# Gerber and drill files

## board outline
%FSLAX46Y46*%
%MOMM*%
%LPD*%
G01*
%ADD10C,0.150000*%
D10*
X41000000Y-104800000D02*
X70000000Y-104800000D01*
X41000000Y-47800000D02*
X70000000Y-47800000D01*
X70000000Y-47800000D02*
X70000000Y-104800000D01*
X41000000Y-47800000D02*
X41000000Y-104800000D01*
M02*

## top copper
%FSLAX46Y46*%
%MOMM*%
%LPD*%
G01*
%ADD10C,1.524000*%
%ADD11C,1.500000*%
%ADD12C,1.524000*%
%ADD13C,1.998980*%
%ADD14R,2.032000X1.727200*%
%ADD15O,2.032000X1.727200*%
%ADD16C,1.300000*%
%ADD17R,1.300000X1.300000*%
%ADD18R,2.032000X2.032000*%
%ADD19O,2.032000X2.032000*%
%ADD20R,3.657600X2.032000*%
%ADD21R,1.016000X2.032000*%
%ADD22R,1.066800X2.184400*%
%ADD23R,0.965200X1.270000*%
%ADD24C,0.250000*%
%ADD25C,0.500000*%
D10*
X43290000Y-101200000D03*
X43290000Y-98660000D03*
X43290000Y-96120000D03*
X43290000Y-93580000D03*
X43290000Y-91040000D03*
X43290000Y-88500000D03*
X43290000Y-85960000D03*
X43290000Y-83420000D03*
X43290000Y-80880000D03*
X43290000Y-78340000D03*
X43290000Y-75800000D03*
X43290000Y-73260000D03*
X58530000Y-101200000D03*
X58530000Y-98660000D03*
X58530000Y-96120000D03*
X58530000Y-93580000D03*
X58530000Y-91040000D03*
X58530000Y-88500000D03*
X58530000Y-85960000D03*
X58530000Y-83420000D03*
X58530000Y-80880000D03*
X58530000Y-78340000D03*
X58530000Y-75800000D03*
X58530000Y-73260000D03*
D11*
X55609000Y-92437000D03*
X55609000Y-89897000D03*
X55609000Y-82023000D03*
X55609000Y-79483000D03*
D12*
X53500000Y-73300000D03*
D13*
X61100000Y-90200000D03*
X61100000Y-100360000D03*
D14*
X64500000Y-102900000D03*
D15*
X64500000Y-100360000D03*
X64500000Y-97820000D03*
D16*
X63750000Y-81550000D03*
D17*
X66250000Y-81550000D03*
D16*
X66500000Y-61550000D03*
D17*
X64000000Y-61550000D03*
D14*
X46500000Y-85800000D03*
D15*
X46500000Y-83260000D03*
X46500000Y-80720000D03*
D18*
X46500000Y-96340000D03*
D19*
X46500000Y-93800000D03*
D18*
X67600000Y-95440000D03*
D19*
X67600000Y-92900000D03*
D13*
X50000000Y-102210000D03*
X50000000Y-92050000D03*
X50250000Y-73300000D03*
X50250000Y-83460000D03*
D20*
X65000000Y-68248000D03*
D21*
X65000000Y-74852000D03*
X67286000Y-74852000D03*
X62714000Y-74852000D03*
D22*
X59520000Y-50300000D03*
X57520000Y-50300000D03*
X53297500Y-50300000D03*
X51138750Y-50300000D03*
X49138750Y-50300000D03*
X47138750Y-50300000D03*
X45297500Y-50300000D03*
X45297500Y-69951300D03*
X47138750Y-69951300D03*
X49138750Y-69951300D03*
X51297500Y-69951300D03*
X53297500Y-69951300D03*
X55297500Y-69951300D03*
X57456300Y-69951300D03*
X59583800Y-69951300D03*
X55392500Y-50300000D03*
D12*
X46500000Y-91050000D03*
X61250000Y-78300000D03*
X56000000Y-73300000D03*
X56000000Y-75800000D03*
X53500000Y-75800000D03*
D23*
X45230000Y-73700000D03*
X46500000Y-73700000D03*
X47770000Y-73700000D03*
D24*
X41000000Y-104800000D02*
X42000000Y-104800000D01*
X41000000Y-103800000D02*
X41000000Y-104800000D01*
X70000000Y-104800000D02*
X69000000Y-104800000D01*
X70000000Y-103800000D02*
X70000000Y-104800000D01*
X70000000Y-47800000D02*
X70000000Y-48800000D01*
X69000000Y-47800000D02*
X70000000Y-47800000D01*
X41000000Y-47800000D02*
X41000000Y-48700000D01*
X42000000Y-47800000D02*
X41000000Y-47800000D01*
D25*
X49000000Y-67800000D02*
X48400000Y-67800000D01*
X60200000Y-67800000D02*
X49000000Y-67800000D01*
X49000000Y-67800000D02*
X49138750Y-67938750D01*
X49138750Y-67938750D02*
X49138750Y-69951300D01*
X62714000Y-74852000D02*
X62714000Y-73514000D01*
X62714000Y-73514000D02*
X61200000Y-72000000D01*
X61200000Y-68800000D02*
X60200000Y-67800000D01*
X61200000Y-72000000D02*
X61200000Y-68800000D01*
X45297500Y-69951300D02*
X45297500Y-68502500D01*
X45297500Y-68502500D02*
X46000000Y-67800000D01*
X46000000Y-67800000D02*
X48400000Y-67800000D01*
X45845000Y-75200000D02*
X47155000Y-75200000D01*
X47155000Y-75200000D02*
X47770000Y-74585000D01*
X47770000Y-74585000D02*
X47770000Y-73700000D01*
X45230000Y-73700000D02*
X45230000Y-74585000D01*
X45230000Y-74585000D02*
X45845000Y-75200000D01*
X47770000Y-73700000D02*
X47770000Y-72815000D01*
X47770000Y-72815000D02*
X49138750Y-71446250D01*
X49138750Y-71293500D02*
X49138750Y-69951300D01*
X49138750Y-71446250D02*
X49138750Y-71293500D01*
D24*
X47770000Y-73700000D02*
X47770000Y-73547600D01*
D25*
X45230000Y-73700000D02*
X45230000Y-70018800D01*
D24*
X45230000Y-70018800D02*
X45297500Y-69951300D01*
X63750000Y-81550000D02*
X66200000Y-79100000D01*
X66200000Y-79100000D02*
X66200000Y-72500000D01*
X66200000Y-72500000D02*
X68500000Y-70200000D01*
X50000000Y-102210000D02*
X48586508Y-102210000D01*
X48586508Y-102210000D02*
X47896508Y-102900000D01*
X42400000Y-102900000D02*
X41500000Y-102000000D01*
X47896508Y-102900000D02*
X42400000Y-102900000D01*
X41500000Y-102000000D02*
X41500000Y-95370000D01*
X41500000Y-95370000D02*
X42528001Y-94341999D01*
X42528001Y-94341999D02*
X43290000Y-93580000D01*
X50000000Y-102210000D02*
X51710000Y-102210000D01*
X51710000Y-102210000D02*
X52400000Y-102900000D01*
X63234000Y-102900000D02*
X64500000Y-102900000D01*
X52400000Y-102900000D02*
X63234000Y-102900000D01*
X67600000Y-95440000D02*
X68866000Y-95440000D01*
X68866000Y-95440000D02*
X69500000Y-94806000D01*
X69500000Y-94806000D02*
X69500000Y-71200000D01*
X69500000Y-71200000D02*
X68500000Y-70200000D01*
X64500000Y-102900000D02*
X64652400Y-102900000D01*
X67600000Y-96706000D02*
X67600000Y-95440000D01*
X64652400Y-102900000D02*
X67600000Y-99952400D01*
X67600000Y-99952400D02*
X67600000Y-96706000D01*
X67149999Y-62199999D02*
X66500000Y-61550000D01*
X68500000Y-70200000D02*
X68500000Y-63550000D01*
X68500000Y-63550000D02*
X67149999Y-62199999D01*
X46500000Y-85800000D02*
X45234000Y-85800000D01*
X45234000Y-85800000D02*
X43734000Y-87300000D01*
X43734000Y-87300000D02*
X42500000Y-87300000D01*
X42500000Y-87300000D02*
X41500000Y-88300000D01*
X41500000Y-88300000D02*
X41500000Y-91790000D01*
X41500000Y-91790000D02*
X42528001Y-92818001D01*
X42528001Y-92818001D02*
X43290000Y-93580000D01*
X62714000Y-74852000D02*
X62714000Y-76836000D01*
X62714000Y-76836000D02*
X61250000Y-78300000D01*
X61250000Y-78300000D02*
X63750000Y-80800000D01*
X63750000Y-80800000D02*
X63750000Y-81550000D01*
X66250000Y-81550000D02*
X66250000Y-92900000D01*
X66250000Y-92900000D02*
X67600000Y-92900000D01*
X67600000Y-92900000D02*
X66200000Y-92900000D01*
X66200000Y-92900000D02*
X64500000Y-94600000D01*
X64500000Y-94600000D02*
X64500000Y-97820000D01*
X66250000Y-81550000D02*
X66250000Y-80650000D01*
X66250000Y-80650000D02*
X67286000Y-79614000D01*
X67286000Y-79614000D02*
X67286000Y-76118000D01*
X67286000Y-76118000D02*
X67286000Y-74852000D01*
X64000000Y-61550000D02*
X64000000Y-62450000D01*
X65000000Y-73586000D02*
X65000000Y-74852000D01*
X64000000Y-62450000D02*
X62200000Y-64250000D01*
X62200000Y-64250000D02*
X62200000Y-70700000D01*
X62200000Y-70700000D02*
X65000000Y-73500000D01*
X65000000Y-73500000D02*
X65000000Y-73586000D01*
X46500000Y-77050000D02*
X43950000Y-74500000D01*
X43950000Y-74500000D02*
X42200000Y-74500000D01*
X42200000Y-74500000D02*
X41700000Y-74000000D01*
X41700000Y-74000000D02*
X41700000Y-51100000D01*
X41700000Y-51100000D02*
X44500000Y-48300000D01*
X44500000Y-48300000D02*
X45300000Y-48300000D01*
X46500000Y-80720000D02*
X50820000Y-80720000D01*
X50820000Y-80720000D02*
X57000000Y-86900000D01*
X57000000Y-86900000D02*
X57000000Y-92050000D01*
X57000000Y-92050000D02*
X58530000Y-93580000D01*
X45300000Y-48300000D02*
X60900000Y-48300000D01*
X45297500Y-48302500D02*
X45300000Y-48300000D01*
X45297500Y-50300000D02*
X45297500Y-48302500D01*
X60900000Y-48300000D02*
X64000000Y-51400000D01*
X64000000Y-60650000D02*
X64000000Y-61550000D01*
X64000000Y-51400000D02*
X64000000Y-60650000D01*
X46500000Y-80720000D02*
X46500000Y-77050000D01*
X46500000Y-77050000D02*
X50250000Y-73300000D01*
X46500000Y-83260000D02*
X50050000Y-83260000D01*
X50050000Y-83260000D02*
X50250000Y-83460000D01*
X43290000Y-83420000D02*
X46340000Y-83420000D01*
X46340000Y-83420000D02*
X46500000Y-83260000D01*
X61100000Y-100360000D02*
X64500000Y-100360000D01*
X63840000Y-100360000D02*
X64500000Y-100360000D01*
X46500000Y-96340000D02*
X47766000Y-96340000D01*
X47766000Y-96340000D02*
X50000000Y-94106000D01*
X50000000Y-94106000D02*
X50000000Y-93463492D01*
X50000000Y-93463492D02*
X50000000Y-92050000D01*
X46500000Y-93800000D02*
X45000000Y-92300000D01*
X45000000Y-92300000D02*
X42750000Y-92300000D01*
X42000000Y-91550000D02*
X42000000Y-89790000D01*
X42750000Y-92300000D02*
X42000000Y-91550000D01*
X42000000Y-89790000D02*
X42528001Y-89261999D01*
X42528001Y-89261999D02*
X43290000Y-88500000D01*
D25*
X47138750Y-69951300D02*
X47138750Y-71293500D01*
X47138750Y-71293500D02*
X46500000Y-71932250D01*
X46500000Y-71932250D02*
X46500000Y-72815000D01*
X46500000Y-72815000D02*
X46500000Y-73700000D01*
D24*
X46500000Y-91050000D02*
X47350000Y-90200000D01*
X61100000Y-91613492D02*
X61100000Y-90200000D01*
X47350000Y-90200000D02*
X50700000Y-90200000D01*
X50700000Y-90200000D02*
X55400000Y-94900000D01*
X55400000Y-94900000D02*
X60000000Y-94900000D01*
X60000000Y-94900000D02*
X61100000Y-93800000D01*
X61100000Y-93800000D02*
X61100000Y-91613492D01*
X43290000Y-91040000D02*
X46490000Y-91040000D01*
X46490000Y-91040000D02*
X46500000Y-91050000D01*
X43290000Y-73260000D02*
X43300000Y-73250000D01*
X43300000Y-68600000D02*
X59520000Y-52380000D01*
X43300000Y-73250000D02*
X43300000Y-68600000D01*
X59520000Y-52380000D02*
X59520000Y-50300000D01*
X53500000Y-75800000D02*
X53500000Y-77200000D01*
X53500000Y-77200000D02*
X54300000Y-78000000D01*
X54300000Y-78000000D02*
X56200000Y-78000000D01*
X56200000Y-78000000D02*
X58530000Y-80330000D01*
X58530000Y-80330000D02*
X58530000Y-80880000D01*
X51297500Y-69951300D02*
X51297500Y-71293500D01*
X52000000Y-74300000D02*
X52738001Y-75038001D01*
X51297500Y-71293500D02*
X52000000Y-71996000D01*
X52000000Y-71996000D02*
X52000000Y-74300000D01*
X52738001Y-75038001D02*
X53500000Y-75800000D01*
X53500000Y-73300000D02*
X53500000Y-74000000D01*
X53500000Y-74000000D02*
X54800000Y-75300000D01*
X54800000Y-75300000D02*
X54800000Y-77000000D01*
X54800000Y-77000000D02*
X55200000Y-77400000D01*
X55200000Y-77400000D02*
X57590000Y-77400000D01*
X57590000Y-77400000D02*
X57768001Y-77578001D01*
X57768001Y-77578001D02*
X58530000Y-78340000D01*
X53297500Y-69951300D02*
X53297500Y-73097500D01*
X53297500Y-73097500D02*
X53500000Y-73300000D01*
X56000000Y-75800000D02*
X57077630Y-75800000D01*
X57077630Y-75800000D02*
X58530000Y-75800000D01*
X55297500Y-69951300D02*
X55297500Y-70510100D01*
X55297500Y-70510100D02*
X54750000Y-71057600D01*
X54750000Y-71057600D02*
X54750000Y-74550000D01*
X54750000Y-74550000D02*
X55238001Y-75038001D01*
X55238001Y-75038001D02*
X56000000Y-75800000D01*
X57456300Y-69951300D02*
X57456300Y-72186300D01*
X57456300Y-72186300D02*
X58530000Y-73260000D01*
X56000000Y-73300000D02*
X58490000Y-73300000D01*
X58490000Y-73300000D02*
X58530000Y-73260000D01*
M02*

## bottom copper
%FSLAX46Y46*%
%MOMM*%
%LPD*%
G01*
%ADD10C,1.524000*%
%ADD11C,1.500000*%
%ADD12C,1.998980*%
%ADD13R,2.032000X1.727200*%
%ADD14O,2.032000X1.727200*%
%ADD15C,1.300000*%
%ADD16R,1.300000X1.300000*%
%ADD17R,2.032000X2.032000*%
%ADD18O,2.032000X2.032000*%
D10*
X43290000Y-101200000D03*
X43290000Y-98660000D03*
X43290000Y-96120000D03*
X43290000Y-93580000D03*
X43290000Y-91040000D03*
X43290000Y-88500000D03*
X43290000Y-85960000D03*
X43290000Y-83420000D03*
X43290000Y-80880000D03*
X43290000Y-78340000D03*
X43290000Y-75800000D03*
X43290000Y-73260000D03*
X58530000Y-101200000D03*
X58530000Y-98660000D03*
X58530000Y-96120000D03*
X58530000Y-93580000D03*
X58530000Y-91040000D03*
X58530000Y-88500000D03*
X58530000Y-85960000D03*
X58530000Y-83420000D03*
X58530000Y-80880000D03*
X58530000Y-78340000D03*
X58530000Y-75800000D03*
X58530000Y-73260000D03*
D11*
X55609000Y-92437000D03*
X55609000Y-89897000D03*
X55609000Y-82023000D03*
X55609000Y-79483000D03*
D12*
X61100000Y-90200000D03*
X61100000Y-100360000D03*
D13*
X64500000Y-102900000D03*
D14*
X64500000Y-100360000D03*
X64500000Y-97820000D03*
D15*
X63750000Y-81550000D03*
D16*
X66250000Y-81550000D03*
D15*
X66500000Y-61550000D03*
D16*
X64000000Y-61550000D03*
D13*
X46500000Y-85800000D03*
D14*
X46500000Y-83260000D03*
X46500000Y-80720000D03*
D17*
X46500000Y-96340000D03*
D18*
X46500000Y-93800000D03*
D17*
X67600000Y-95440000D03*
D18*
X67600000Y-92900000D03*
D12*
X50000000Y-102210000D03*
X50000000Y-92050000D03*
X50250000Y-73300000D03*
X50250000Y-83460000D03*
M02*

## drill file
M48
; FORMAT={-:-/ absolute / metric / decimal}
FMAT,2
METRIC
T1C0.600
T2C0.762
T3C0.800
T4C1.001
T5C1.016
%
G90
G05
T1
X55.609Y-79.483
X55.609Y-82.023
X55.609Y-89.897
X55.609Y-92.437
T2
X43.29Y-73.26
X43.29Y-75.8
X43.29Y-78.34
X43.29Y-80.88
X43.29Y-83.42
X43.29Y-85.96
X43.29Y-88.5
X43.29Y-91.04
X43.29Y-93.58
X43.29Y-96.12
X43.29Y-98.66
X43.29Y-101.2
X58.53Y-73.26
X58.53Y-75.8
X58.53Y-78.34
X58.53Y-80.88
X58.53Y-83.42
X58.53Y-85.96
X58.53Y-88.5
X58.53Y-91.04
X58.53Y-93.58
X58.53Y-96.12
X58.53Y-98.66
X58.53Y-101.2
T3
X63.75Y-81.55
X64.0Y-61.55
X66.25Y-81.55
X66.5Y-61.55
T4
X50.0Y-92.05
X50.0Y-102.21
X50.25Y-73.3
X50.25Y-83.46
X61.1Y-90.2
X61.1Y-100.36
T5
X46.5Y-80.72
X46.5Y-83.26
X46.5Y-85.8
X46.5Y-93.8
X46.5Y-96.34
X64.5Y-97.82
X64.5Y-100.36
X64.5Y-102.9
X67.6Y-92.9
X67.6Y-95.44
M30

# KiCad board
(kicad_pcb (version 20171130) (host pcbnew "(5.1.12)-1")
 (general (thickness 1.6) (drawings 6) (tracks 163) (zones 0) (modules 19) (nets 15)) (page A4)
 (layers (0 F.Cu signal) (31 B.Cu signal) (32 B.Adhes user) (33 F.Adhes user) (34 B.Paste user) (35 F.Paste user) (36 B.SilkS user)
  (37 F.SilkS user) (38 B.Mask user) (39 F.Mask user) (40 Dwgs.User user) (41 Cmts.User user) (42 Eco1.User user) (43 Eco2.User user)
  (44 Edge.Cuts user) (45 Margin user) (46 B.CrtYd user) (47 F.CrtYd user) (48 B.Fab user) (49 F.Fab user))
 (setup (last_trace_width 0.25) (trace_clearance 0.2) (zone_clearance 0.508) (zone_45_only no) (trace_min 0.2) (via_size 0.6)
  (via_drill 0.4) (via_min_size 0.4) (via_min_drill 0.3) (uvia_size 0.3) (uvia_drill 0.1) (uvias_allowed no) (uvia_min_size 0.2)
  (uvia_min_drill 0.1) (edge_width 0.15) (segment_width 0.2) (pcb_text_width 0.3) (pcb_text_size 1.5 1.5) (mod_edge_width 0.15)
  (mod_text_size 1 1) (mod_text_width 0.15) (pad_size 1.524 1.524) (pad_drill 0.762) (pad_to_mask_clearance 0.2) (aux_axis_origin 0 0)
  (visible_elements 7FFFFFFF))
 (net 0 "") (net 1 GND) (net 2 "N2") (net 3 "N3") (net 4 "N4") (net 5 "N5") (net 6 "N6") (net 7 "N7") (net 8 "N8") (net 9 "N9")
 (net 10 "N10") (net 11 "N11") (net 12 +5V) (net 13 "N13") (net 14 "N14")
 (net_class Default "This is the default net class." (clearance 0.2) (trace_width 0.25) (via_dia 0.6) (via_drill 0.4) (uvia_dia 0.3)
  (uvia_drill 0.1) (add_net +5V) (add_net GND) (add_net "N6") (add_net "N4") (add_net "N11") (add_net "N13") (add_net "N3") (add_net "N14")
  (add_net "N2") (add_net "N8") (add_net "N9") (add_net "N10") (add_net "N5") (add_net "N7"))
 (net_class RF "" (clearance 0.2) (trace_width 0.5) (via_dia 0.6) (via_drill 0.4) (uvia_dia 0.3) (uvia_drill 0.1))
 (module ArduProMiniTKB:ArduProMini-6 (layer B.Cu) (at 40.75 107.55)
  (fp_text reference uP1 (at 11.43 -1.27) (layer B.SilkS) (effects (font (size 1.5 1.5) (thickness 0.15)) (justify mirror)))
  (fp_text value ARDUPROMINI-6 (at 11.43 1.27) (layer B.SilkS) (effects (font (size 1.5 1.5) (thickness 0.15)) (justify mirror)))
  (pad 7 thru_hole circle (at 2.54 -6.35) (size 1.524 1.524) (drill 0.762) (layers *.Cu *.Mask B.SilkS))
  (pad 8 thru_hole circle (at 2.54 -8.89) (size 1.524 1.524) (drill 0.762) (layers *.Cu *.Mask B.SilkS))
  (pad 9 thru_hole circle (at 2.54 -11.43) (size 1.524 1.524) (drill 0.762) (layers *.Cu *.Mask B.SilkS))
  (pad 10 thru_hole circle (at 2.54 -13.97) (size 1.524 1.524) (drill 0.762) (layers *.Cu *.Mask B.SilkS) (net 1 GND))
  (pad 11 thru_hole circle (at 2.54 -16.51) (size 1.524 1.524) (drill 0.762) (layers *.Cu *.Mask B.SilkS) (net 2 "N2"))
  (pad 12 thru_hole circle (at 2.54 -19.05) (size 1.524 1.524) (drill 0.762) (layers *.Cu *.Mask B.SilkS) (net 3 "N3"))
  (pad 13 thru_hole circle (at 2.54 -21.59) (size 1.524 1.524) (drill 0.762) (layers *.Cu *.Mask B.SilkS))
  (pad 14 thru_hole circle (at 2.54 -24.13) (size 1.524 1.524) (drill 0.762) (layers *.Cu *.Mask B.SilkS) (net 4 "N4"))
  (pad 15 thru_hole circle (at 2.54 -26.67) (size 1.524 1.524) (drill 0.762) (layers *.Cu *.Mask B.SilkS))
  (pad 16 thru_hole circle (at 2.54 -29.21) (size 1.524 1.524) (drill 0.762) (layers *.Cu *.Mask B.SilkS))
  (pad 17 thru_hole circle (at 2.54 -31.75) (size 1.524 1.524) (drill 0.762) (layers *.Cu *.Mask B.SilkS))
  (pad 18 thru_hole circle (at 2.54 -34.29) (size 1.524 1.524) (drill 0.762) (layers *.Cu *.Mask B.SilkS) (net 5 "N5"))
  (pad 19 thru_hole circle (at 17.78 -6.35) (size 1.524 1.524) (drill 0.762) (layers *.Cu *.Mask B.SilkS))
  (pad 20 thru_hole circle (at 17.78 -8.89) (size 1.524 1.524) (drill 0.762) (layers *.Cu *.Mask B.SilkS))
  (pad 21 thru_hole circle (at 17.78 -11.43) (size 1.524 1.524) (drill 0.762) (layers *.Cu *.Mask B.SilkS))
  (pad 22 thru_hole circle (at 17.78 -13.97) (size 1.524 1.524) (drill 0.762) (layers *.Cu *.Mask B.SilkS) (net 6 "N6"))
  (pad 23 thru_hole circle (at 17.78 -16.51) (size 1.524 1.524) (drill 0.762) (layers *.Cu *.Mask B.SilkS))
  (pad 24 thru_hole circle (at 17.78 -19.05) (size 1.524 1.524) (drill 0.762) (layers *.Cu *.Mask B.SilkS))
  (pad 25 thru_hole circle (at 17.78 -21.59) (size 1.524 1.524) (drill 0.762) (layers *.Cu *.Mask B.SilkS))
  (pad 26 thru_hole circle (at 17.78 -24.13) (size 1.524 1.524) (drill 0.762) (layers *.Cu *.Mask B.SilkS))
  (pad 27 thru_hole circle (at 17.78 -26.67) (size 1.524 1.524) (drill 0.762) (layers *.Cu *.Mask B.SilkS) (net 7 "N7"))
  (pad 28 thru_hole circle (at 17.78 -29.21) (size 1.524 1.524) (drill 0.762) (layers *.Cu *.Mask B.SilkS) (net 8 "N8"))
  (pad 29 thru_hole circle (at 17.78 -31.75) (size 1.524 1.524) (drill 0.762) (layers *.Cu *.Mask B.SilkS) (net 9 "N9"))
  (pad 30 thru_hole circle (at 17.78 -34.29) (size 1.524 1.524) (drill 0.762) (layers *.Cu *.Mask B.SilkS) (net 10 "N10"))
  (pad 31 thru_hole circle (at 14.859 -15.113) (size 1.5 1.5) (drill 0.6) (layers *.Cu *.Mask B.SilkS))
  (pad 32 thru_hole circle (at 14.859 -17.653) (size 1.5 1.5) (drill 0.6) (layers *.Cu *.Mask B.SilkS))
  (pad 34 thru_hole circle (at 14.859 -25.527) (size 1.5 1.5) (drill 0.6) (layers *.Cu *.Mask B.SilkS))
  (pad 35 thru_hole circle (at 14.859 -28.067) (size 1.5 1.5) (drill 0.6) (layers *.Cu *.Mask B.SilkS)))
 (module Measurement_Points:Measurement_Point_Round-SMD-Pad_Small (layer F.Cu) (at 53.5 73.3)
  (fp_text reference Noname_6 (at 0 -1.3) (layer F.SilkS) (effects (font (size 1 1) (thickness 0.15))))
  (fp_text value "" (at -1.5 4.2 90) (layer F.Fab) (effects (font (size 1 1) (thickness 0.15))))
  (pad 1 smd circle (at 0 0) (size 1.524 1.524) (layers F.Cu F.Paste F.Mask) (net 8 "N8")))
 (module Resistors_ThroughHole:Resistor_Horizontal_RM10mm (layer F.Cu) (at 61.1 90.2 270)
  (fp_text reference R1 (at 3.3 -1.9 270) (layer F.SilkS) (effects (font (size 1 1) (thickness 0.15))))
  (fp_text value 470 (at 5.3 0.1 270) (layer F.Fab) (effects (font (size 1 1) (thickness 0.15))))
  (pad 1 thru_hole circle (at 0 0 270) (size 1.99898 1.99898) (drill 1.00076) (layers *.Cu *.SilkS *.Mask) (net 2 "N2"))
  (pad 2 thru_hole circle (at 10.16 0 270) (size 1.99898 1.99898) (drill 1.00076) (layers *.Cu *.SilkS *.Mask) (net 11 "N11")))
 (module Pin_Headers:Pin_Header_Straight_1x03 (layer F.Cu) (at 64.5 102.9 180)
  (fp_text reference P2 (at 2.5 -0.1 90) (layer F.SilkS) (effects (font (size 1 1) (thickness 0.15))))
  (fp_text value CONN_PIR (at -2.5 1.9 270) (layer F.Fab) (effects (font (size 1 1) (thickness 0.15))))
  (pad 1 thru_hole rect (at 0 0 180) (size 2.032 1.7272) (drill 1.016) (layers *.Cu *.Mask F.SilkS) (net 1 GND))
  (pad 2 thru_hole oval (at 0 2.54 180) (size 2.032 1.7272) (drill 1.016) (layers *.Cu *.Mask F.SilkS) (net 11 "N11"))
  (pad 3 thru_hole oval (at 0 5.08 180) (size 2.032 1.7272) (drill 1.016) (layers *.Cu *.Mask F.SilkS) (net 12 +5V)))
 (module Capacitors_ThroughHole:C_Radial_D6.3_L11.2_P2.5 (layer F.Cu) (at 66.25 81.55 180)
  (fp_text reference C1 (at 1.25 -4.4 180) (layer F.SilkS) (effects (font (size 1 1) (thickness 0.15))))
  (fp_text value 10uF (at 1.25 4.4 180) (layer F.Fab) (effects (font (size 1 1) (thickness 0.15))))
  (pad 2 thru_hole circle (at 2.5 0 180) (size 1.3 1.3) (drill 0.8) (layers *.Cu *.Mask F.SilkS) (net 1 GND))
  (pad 1 thru_hole rect (at 0 0 180) (size 1.3 1.3) (drill 0.8) (layers *.Cu *.Mask F.SilkS) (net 12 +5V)))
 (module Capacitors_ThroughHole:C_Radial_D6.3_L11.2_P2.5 (layer F.Cu) (at 64 61.55)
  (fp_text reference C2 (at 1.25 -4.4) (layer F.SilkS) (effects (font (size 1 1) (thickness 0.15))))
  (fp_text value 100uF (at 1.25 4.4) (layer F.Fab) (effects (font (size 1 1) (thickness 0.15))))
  (pad 2 thru_hole circle (at 2.5 0) (size 1.3 1.3) (drill 0.8) (layers *.Cu *.Mask F.SilkS) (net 1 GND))
  (pad 1 thru_hole rect (at 0 0) (size 1.3 1.3) (drill 0.8) (layers *.Cu *.Mask F.SilkS) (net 6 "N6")))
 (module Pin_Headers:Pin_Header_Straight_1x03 (layer F.Cu) (at 46.5 85.8 180)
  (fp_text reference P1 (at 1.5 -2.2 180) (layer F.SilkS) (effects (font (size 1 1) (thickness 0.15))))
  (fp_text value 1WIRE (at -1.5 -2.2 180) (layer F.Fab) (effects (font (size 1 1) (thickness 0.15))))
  (pad 1 thru_hole rect (at 0 0 180) (size 2.032 1.7272) (drill 1.016) (layers *.Cu *.Mask F.SilkS) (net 1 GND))
  (pad 2 thru_hole oval (at 0 2.54 180) (size 2.032 1.7272) (drill 1.016) (layers *.Cu *.Mask F.SilkS) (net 4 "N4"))
  (pad 3 thru_hole oval (at 0 5.08 180) (size 2.032 1.7272) (drill 1.016) (layers *.Cu *.Mask F.SilkS) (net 6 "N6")))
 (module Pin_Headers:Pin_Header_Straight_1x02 (layer F.Cu) (at 46.5 96.34 180)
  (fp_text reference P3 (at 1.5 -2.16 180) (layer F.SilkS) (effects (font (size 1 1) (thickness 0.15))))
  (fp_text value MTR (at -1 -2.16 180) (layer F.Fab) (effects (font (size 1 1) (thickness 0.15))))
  (pad 1 thru_hole rect (at 0 0 180) (size 2.032 2.032) (drill 1.016) (layers *.Cu *.Mask F.SilkS) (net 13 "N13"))
  (pad 2 thru_hole oval (at 0 2.54 180) (size 2.032 2.032) (drill 1.016) (layers *.Cu *.Mask F.SilkS) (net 3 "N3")))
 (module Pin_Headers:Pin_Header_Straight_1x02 (layer F.Cu) (at 67.6 95.44 180)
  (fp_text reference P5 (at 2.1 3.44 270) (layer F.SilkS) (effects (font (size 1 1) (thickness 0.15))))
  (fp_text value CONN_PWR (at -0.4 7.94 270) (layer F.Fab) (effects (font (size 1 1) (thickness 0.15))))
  (pad 1 thru_hole rect (at 0 0 180) (size 2.032 2.032) (drill 1.016) (layers *.Cu *.Mask F.SilkS) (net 1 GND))
  (pad 2 thru_hole oval (at 0 2.54 180) (size 2.032 2.032) (drill 1.016) (layers *.Cu *.Mask F.SilkS) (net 12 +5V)))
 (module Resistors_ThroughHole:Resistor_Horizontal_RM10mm (layer F.Cu) (at 50 102.21 90)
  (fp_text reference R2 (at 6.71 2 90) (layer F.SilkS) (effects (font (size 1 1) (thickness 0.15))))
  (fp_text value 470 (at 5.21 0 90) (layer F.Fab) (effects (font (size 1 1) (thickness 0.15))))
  (pad 1 thru_hole circle (at 0 0 90) (size 1.99898 1.99898) (drill 1.00076) (layers *.Cu *.SilkS *.Mask) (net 1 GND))
  (pad 2 thru_hole circle (at 10.16 0 90) (size 1.99898 1.99898) (drill 1.00076) (layers *.Cu *.SilkS *.Mask) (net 13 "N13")))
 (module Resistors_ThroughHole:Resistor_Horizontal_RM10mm (layer F.Cu) (at 50.25 73.3 270)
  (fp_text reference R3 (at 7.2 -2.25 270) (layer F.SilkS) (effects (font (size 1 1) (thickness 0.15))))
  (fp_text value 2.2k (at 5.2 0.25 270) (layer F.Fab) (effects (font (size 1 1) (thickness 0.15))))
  (pad 1 thru_hole circle (at 0 0 270) (size 1.99898 1.99898) (drill 1.00076) (layers *.Cu *.SilkS *.Mask) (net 6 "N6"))
  (pad 2 thru_hole circle (at 10.16 0 270) (size 1.99898 1.99898) (drill 1.00076) (layers *.Cu *.SilkS *.Mask) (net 4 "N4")))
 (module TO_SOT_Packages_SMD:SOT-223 (layer F.Cu) (at 65 71.55)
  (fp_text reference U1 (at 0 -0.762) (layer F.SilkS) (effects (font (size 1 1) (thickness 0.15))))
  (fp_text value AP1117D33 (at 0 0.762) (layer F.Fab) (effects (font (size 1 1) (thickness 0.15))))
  (pad 4 smd rect (at 0 -3.302) (size 3.6576 2.032) (layers F.Cu F.Paste F.Mask))
  (pad 2 smd rect (at 0 3.302) (size 1.016 2.032) (layers F.Cu F.Paste F.Mask) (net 6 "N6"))
  (pad 3 smd rect (at 2.286 3.302) (size 1.016 2.032) (layers F.Cu F.Paste F.Mask) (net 12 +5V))
  (pad 1 smd rect (at -2.286 3.302) (size 1.016 2.032) (layers F.Cu F.Paste F.Mask) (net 1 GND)))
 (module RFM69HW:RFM (layer F.Cu) (at 44.25 50.3 270) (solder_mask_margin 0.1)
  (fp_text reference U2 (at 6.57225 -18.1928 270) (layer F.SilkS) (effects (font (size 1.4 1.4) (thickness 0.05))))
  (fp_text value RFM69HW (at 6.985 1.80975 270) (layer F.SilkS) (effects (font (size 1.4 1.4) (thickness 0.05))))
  (pad RESE smd rect (at 0 -15.27 270) (size 2.1844 1.0668) (layers F.Cu F.Paste F.Mask) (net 5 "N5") (solder_mask_margin 0.2))
  (pad DIO0 smd rect (at 0 -13.27 270) (size 2.1844 1.0668) (layers F.Cu F.Paste F.Mask) (solder_mask_margin 0.2))
  (pad DIO2 smd rect (at 0 -9.0475 270) (size 2.1844 1.0668) (layers F.Cu F.Paste F.Mask) (solder_mask_margin 0.2))
  (pad DIO3 smd rect (at 0 -6.88875 270) (size 2.1844 1.0668) (layers F.Cu F.Paste F.Mask) (solder_mask_margin 0.2))
  (pad DIO4 smd rect (at 0 -4.88875 270) (size 2.1844 1.0668) (layers F.Cu F.Paste F.Mask) (solder_mask_margin 0.2))
  (pad DIO5 smd rect (at 0 -2.88875 270) (size 2.1844 1.0668) (layers F.Cu F.Paste F.Mask) (solder_mask_margin 0.2))
  (pad VCC smd rect (at 0 -1.0475 270) (size 2.1844 1.0668) (layers F.Cu F.Paste F.Mask) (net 6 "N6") (solder_mask_margin 0.2))
  (pad GNDB smd rect (at 19.6513 -1.0475 270) (size 2.1844 1.0668) (layers F.Cu F.Paste F.Mask) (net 1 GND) (solder_mask_margin 0.2))
  (pad ANT smd rect (at 19.6513 -2.88875 270) (size 2.1844 1.0668) (layers F.Cu F.Paste F.Mask) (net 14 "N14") (solder_mask_margin 0.2))
  (pad GNDA smd rect (at 19.6513 -4.88875 270) (size 2.1844 1.0668) (layers F.Cu F.Paste F.Mask) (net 1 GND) (solder_mask_margin 0.2))
  (pad SCK smd rect (at 19.6513 -7.0475 270) (size 2.1844 1.0668) (layers F.Cu F.Paste F.Mask) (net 7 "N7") (solder_mask_margin 0.2))
  (pad MISO smd rect (at 19.6513 -9.0475 270) (size 2.1844 1.0668) (layers F.Cu F.Paste F.Mask) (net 8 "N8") (solder_mask_margin 0.2))
  (pad MOSI smd rect (at 19.6513 -11.0475 270) (size 2.1844 1.0668) (layers F.Cu F.Paste F.Mask) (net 9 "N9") (solder_mask_margin 0.2))
  (pad NSS smd rect (at 19.6513 -13.2063 270) (size 2.1844 1.0668) (layers F.Cu F.Paste F.Mask) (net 10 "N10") (solder_mask_margin 0.2))
  (pad NC smd rect (at 19.6513 -15.3338 270) (size 2.1844 1.0668) (layers F.Cu F.Paste F.Mask) (solder_mask_margin 0.2))
  (pad DIO1 smd rect (at 0 -11.1425 270) (size 2.1844 1.0668) (layers F.Cu F.Paste F.Mask) (solder_mask_margin 0.2)))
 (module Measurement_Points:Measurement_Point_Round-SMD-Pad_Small (layer F.Cu) (at 46.5 91.05)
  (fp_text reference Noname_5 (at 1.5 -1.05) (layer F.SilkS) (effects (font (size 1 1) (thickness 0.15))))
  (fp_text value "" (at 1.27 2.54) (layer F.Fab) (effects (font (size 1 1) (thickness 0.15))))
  (pad 1 smd circle (at 0 0) (size 1.524 1.524) (layers F.Cu F.Paste F.Mask) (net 2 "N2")))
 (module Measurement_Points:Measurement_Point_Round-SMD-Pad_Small (layer F.Cu) (at 61.25 78.3)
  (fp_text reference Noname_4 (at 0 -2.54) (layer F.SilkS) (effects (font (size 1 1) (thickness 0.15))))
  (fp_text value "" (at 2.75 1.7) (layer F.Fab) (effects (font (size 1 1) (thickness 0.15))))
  (pad 1 smd circle (at 0 0) (size 1.524 1.524) (layers F.Cu F.Paste F.Mask) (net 1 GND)))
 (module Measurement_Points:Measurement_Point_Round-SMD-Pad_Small (layer F.Cu) (at 56 73.3)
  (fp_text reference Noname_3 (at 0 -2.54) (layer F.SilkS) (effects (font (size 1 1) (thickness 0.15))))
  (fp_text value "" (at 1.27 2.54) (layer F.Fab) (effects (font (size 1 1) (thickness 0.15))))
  (pad 1 smd circle (at 0 0) (size 1.524 1.524) (layers F.Cu F.Paste F.Mask) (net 10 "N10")))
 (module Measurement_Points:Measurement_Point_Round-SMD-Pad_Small (layer F.Cu) (at 56 75.8)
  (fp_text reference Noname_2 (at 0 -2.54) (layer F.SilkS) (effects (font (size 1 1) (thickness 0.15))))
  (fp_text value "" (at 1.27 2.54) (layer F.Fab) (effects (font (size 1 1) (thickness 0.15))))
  (pad 1 smd circle (at 0 0) (size 1.524 1.524) (layers F.Cu F.Paste F.Mask) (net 9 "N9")))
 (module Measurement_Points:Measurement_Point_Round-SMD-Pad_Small (layer F.Cu) (at 53.5 75.8)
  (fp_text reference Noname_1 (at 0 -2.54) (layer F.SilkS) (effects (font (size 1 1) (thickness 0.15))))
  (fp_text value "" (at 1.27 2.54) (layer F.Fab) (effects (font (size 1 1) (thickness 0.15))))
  (pad 1 smd circle (at 0 0) (size 1.524 1.524) (layers F.Cu F.Paste F.Mask) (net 7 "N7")))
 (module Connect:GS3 (layer F.Cu) (at 46.5 73.7 90)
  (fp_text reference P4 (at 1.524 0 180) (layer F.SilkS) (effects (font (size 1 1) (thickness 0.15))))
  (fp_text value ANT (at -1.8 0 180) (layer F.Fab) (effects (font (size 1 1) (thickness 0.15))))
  (pad 1 smd rect (at 0 -1.27 90) (size 1.27 0.9652) (layers F.Cu F.Paste F.Mask) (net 1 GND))
  (pad 2 smd rect (at 0 0 90) (size 1.27 0.9652) (layers F.Cu F.Paste F.Mask) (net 14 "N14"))
  (pad 3 smd rect (at 0 1.27 90) (size 1.27 0.9652) (layers F.Cu F.Paste F.Mask) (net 1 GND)))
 (gr_line (start 41 104.8) (end 70 104.8) (angle 90) (layer Edge.Cuts) (width 0.15))
 (gr_line (start 41 47.8) (end 70 47.8) (angle 90) (layer Edge.Cuts) (width 0.15))
 (gr_line (start 70 47.8) (end 70 104.8) (angle 90) (layer Edge.Cuts) (width 0.15))
 (gr_line (start 41 47.8) (end 41 104.8) (angle 90) (layer Edge.Cuts) (width 0.15))
 (segment (start 41 104.8) (end 42 104.8) (width 0.25) (layer F.Cu) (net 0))
 (segment (start 41 103.8) (end 41 104.8) (width 0.25) (layer F.Cu) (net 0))
 (segment (start 70 104.8) (end 69 104.8) (width 0.25) (layer F.Cu) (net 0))
 (segment (start 70 103.8) (end 70 104.8) (width 0.25) (layer F.Cu) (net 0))
 (segment (start 70 47.8) (end 70 48.8) (width 0.25) (layer F.Cu) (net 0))
 (segment (start 69 47.8) (end 70 47.8) (width 0.25) (layer F.Cu) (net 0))
 (segment (start 41 47.8) (end 41 48.7) (width 0.25) (layer F.Cu) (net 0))
 (segment (start 42 47.8) (end 41 47.8) (width 0.25) (layer F.Cu) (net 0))
 (segment (start 49 67.8) (end 48.4 67.8) (width 0.5) (layer F.Cu) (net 1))
 (segment (start 60.2 67.8) (end 49 67.8) (width 0.5) (layer F.Cu) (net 1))
 (segment (start 49 67.8) (end 49.13875 67.93875) (width 0.5) (layer F.Cu) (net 1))
 (segment (start 49.13875 67.93875) (end 49.13875 69.9513) (width 0.5) (layer F.Cu) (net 1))
 (segment (start 62.714 74.852) (end 62.714 73.514) (width 0.5) (layer F.Cu) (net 1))
 (segment (start 62.714 73.514) (end 61.2 72) (width 0.5) (layer F.Cu) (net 1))
 (segment (start 61.2 68.8) (end 60.2 67.8) (width 0.5) (layer F.Cu) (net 1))
 (segment (start 61.2 72) (end 61.2 68.8) (width 0.5) (layer F.Cu) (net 1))
 (segment (start 45.2975 69.9513) (end 45.2975 68.5025) (width 0.5) (layer F.Cu) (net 1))
 (segment (start 45.2975 68.5025) (end 46 67.8) (width 0.5) (layer F.Cu) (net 1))
 (segment (start 46 67.8) (end 48.4 67.8) (width 0.5) (layer F.Cu) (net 1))
 (segment (start 45.845 75.2) (end 47.155 75.2) (width 0.5) (layer F.Cu) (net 1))
 (segment (start 47.155 75.2) (end 47.77 74.585) (width 0.5) (layer F.Cu) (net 1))
 (segment (start 47.77 74.585) (end 47.77 73.7) (width 0.5) (layer F.Cu) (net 1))
 (segment (start 45.23 73.7) (end 45.23 74.585) (width 0.5) (layer F.Cu) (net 1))
 (segment (start 45.23 74.585) (end 45.845 75.2) (width 0.5) (layer F.Cu) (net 1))
 (segment (start 47.77 73.7) (end 47.77 72.815) (width 0.5) (layer F.Cu) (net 1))
 (segment (start 47.77 72.815) (end 49.13875 71.44625) (width 0.5) (layer F.Cu) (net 1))
 (segment (start 49.13875 71.2935) (end 49.13875 69.9513) (width 0.5) (layer F.Cu) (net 1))
 (segment (start 49.13875 71.44625) (end 49.13875 71.2935) (width 0.5) (layer F.Cu) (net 1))
 (segment (start 47.77 73.7) (end 47.77 73.5476) (width 0.25) (layer F.Cu) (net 1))
 (segment (start 45.23 73.7) (end 45.23 70.0188) (width 0.5) (layer F.Cu) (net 1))
 (segment (start 45.23 70.0188) (end 45.2975 69.9513) (width 0.25) (layer F.Cu) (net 1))
 (segment (start 63.75 81.55) (end 66.2 79.1) (width 0.25) (layer F.Cu) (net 1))
 (segment (start 66.2 79.1) (end 66.2 72.5) (width 0.25) (layer F.Cu) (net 1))
 (segment (start 66.2 72.5) (end 68.5 70.2) (width 0.25) (layer F.Cu) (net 1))
 (segment (start 50 102.21) (end 48.586508 102.21) (width 0.25) (layer F.Cu) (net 1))
 (segment (start 48.586508 102.21) (end 47.896508 102.9) (width 0.25) (layer F.Cu) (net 1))
 (segment (start 42.4 102.9) (end 41.5 102) (width 0.25) (layer F.Cu) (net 1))
 (segment (start 47.896508 102.9) (end 42.4 102.9) (width 0.25) (layer F.Cu) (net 1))
 (segment (start 41.5 102) (end 41.5 95.37) (width 0.25) (layer F.Cu) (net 1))
 (segment (start 41.5 95.37) (end 42.528001 94.341999) (width 0.25) (layer F.Cu) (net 1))
 (segment (start 42.528001 94.341999) (end 43.29 93.58) (width 0.25) (layer F.Cu) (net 1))
 (segment (start 50 102.21) (end 51.71 102.21) (width 0.25) (layer F.Cu) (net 1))
 (segment (start 51.71 102.21) (end 52.4 102.9) (width 0.25) (layer F.Cu) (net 1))
 (segment (start 63.234 102.9) (end 64.5 102.9) (width 0.25) (layer F.Cu) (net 1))
 (segment (start 52.4 102.9) (end 63.234 102.9) (width 0.25) (layer F.Cu) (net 1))
 (segment (start 67.6 95.44) (end 68.866 95.44) (width 0.25) (layer F.Cu) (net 1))
 (segment (start 68.866 95.44) (end 69.5 94.806) (width 0.25) (layer F.Cu) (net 1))
 (segment (start 69.5 94.806) (end 69.5 71.2) (width 0.25) (layer F.Cu) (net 1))
 (segment (start 69.5 71.2) (end 68.5 70.2) (width 0.25) (layer F.Cu) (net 1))
 (segment (start 64.5 102.9) (end 64.6524 102.9) (width 0.25) (layer F.Cu) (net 1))
 (segment (start 67.6 96.706) (end 67.6 95.44) (width 0.25) (layer F.Cu) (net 1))
 (segment (start 64.6524 102.9) (end 67.6 99.9524) (width 0.25) (layer F.Cu) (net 1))
 (segment (start 67.6 99.9524) (end 67.6 96.706) (width 0.25) (layer F.Cu) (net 1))
 (segment (start 67.149999 62.199999) (end 66.5 61.55) (width 0.25) (layer F.Cu) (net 1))
 (segment (start 68.5 70.2) (end 68.5 63.55) (width 0.25) (layer F.Cu) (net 1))
 (segment (start 68.5 63.55) (end 67.149999 62.199999) (width 0.25) (layer F.Cu) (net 1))
 (segment (start 46.5 85.8) (end 45.234 85.8) (width 0.25) (layer F.Cu) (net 1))
 (segment (start 45.234 85.8) (end 43.734 87.3) (width 0.25) (layer F.Cu) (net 1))
 (segment (start 43.734 87.3) (end 42.5 87.3) (width 0.25) (layer F.Cu) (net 1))
 (segment (start 42.5 87.3) (end 41.5 88.3) (width 0.25) (layer F.Cu) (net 1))
 (segment (start 41.5 88.3) (end 41.5 91.79) (width 0.25) (layer F.Cu) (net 1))
 (segment (start 41.5 91.79) (end 42.528001 92.818001) (width 0.25) (layer F.Cu) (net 1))
 (segment (start 42.528001 92.818001) (end 43.29 93.58) (width 0.25) (layer F.Cu) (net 1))
 (segment (start 62.714 74.852) (end 62.714 76.836) (width 0.25) (layer F.Cu) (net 1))
 (segment (start 62.714 76.836) (end 61.25 78.3) (width 0.25) (layer F.Cu) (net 1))
 (segment (start 61.25 78.3) (end 63.75 80.8) (width 0.25) (layer F.Cu) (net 1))
 (segment (start 63.75 80.8) (end 63.75 81.55) (width 0.25) (layer F.Cu) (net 1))
 (segment (start 66.25 81.55) (end 66.25 92.9) (width 0.25) (layer F.Cu) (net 12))
 (segment (start 66.25 92.9) (end 67.6 92.9) (width 0.25) (layer F.Cu) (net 12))
 (segment (start 67.6 92.9) (end 66.2 92.9) (width 0.25) (layer F.Cu) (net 12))
 (segment (start 66.2 92.9) (end 64.5 94.6) (width 0.25) (layer F.Cu) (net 12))
 (segment (start 64.5 94.6) (end 64.5 97.82) (width 0.25) (layer F.Cu) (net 12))
 (segment (start 66.25 81.55) (end 66.25 80.65) (width 0.25) (layer F.Cu) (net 12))
 (segment (start 66.25 80.65) (end 67.286 79.614) (width 0.25) (layer F.Cu) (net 12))
 (segment (start 67.286 79.614) (end 67.286 76.118) (width 0.25) (layer F.Cu) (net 12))
 (segment (start 67.286 76.118) (end 67.286 74.852) (width 0.25) (layer F.Cu) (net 12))
 (segment (start 64 61.55) (end 64 62.45) (width 0.25) (layer F.Cu) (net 6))
 (segment (start 65 73.586) (end 65 74.852) (width 0.25) (layer F.Cu) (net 6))
 (segment (start 64 62.45) (end 62.2 64.25) (width 0.25) (layer F.Cu) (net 6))
 (segment (start 62.2 64.25) (end 62.2 70.7) (width 0.25) (layer F.Cu) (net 6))
 (segment (start 62.2 70.7) (end 65 73.5) (width 0.25) (layer F.Cu) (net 6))
 (segment (start 65 73.5) (end 65 73.586) (width 0.25) (layer F.Cu) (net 6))
 (segment (start 46.5 77.05) (end 43.95 74.5) (width 0.25) (layer F.Cu) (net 6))
 (segment (start 43.95 74.5) (end 42.2 74.5) (width 0.25) (layer F.Cu) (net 6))
 (segment (start 42.2 74.5) (end 41.7 74) (width 0.25) (layer F.Cu) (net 6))
 (segment (start 41.7 74) (end 41.7 51.1) (width 0.25) (layer F.Cu) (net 6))
 (segment (start 41.7 51.1) (end 44.5 48.3) (width 0.25) (layer F.Cu) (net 6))
 (segment (start 44.5 48.3) (end 45.3 48.3) (width 0.25) (layer F.Cu) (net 6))
 (segment (start 46.5 80.72) (end 50.82 80.72) (width 0.25) (layer F.Cu) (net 6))
 (segment (start 50.82 80.72) (end 57 86.9) (width 0.25) (layer F.Cu) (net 6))
 (segment (start 57 86.9) (end 57 92.05) (width 0.25) (layer F.Cu) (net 6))
 (segment (start 57 92.05) (end 58.53 93.58) (width 0.25) (layer F.Cu) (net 6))
 (segment (start 45.3 48.3) (end 60.9 48.3) (width 0.25) (layer F.Cu) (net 6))
 (segment (start 45.2975 48.3025) (end 45.3 48.3) (width 0.25) (layer F.Cu) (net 6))
 (segment (start 45.2975 50.3) (end 45.2975 48.3025) (width 0.25) (layer F.Cu) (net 6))
 (segment (start 60.9 48.3) (end 64 51.4) (width 0.25) (layer F.Cu) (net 6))
 (segment (start 64 60.65) (end 64 61.55) (width 0.25) (layer F.Cu) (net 6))
 (segment (start 64 51.4) (end 64 60.65) (width 0.25) (layer F.Cu) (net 6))
 (segment (start 46.5 80.72) (end 46.5 77.05) (width 0.25) (layer F.Cu) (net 6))
 (segment (start 46.5 77.05) (end 50.25 73.3) (width 0.25) (layer F.Cu) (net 6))
 (segment (start 46.5 83.26) (end 50.05 83.26) (width 0.25) (layer F.Cu) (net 4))
 (segment (start 50.05 83.26) (end 50.25 83.46) (width 0.25) (layer F.Cu) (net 4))
 (segment (start 43.29 83.42) (end 46.34 83.42) (width 0.25) (layer F.Cu) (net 4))
 (segment (start 46.34 83.42) (end 46.5 83.26) (width 0.25) (layer F.Cu) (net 4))
 (segment (start 61.1 100.36) (end 64.5 100.36) (width 0.25) (layer F.Cu) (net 11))
 (segment (start 63.84 100.36) (end 64.5 100.36) (width 0.25) (layer F.Cu) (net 11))
 (segment (start 46.5 96.34) (end 47.766 96.34) (width 0.25) (layer F.Cu) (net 13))
 (segment (start 47.766 96.34) (end 50 94.106) (width 0.25) (layer F.Cu) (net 13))
 (segment (start 50 94.106) (end 50 93.463492) (width 0.25) (layer F.Cu) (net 13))
 (segment (start 50 93.463492) (end 50 92.05) (width 0.25) (layer F.Cu) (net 13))
 (segment (start 46.5 93.8) (end 45 92.3) (width 0.25) (layer F.Cu) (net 3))
 (segment (start 45 92.3) (end 42.75 92.3) (width 0.25) (layer F.Cu) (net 3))
 (segment (start 42 91.55) (end 42 89.79) (width 0.25) (layer F.Cu) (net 3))
 (segment (start 42.75 92.3) (end 42 91.55) (width 0.25) (layer F.Cu) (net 3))
 (segment (start 42 89.79) (end 42.528001 89.261999) (width 0.25) (layer F.Cu) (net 3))
 (segment (start 42.528001 89.261999) (end 43.29 88.5) (width 0.25) (layer F.Cu) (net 3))
 (segment (start 47.13875 69.9513) (end 47.13875 71.2935) (width 0.5) (layer F.Cu) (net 14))
 (segment (start 47.13875 71.2935) (end 46.5 71.93225) (width 0.5) (layer F.Cu) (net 14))
 (segment (start 46.5 71.93225) (end 46.5 72.815) (width 0.5) (layer F.Cu) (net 14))
 (segment (start 46.5 72.815) (end 46.5 73.7) (width 0.5) (layer F.Cu) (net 14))
 (segment (start 46.5 91.05) (end 47.35 90.2) (width 0.25) (layer F.Cu) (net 2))
 (segment (start 61.1 91.613492) (end 61.1 90.2) (width 0.25) (layer F.Cu) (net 2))
 (segment (start 47.35 90.2) (end 50.7 90.2) (width 0.25) (layer F.Cu) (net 2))
 (segment (start 50.7 90.2) (end 55.4 94.9) (width 0.25) (layer F.Cu) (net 2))
 (segment (start 55.4 94.9) (end 60 94.9) (width 0.25) (layer F.Cu) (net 2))
 (segment (start 60 94.9) (end 61.1 93.8) (width 0.25) (layer F.Cu) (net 2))
 (segment (start 61.1 93.8) (end 61.1 91.613492) (width 0.25) (layer F.Cu) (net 2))
 (segment (start 43.29 91.04) (end 46.49 91.04) (width 0.25) (layer F.Cu) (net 2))
 (segment (start 46.49 91.04) (end 46.5 91.05) (width 0.25) (layer F.Cu) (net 2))
 (segment (start 43.29 73.26) (end 43.3 73.25) (width 0.25) (layer F.Cu) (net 5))
 (segment (start 43.3 68.6) (end 59.52 52.38) (width 0.25) (layer F.Cu) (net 5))
 (segment (start 43.3 73.25) (end 43.3 68.6) (width 0.25) (layer F.Cu) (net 5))
 (segment (start 59.52 52.38) (end 59.52 50.3) (width 0.25) (layer F.Cu) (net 5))
 (segment (start 53.5 75.8) (end 53.5 77.2) (width 0.25) (layer F.Cu) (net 7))
 (segment (start 53.5 77.2) (end 54.3 78) (width 0.25) (layer F.Cu) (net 7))
 (segment (start 54.3 78) (end 56.2 78) (width 0.25) (layer F.Cu) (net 7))
 (segment (start 56.2 78) (end 58.53 80.33) (width 0.25) (layer F.Cu) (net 7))
 (segment (start 58.53 80.33) (end 58.53 80.88) (width 0.25) (layer F.Cu) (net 7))
 (segment (start 51.2975 69.9513) (end 51.2975 71.2935) (width 0.25) (layer F.Cu) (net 7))
 (segment (start 52 74.3) (end 52.738001 75.038001) (width 0.25) (layer F.Cu) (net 7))
 (segment (start 51.2975 71.2935) (end 52 71.996) (width 0.25) (layer F.Cu) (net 7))
 (segment (start 52 71.996) (end 52 74.3) (width 0.25) (layer F.Cu) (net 7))
 (segment (start 52.738001 75.038001) (end 53.5 75.8) (width 0.25) (layer F.Cu) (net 7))
 (segment (start 53.5 73.3) (end 53.5 74) (width 0.25) (layer F.Cu) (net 8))
 (segment (start 53.5 74) (end 54.8 75.3) (width 0.25) (layer F.Cu) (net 8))
 (segment (start 54.8 75.3) (end 54.8 77) (width 0.25) (layer F.Cu) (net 8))
 (segment (start 54.8 77) (end 55.2 77.4) (width 0.25) (layer F.Cu) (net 8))
 (segment (start 55.2 77.4) (end 57.59 77.4) (width 0.25) (layer F.Cu) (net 8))
 (segment (start 57.59 77.4) (end 57.768001 77.578001) (width 0.25) (layer F.Cu) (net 8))
 (segment (start 57.768001 77.578001) (end 58.53 78.34) (width 0.25) (layer F.Cu) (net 8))
 (segment (start 53.2975 69.9513) (end 53.2975 73.0975) (width 0.25) (layer F.Cu) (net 8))
 (segment (start 53.2975 73.0975) (end 53.5 73.3) (width 0.25) (layer F.Cu) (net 8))
 (segment (start 56 75.8) (end 57.07763 75.8) (width 0.25) (layer F.Cu) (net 9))
 (segment (start 57.07763 75.8) (end 58.53 75.8) (width 0.25) (layer F.Cu) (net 9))
 (segment (start 55.2975 69.9513) (end 55.2975 70.5101) (width 0.25) (layer F.Cu) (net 9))
 (segment (start 55.2975 70.5101) (end 54.75 71.0576) (width 0.25) (layer F.Cu) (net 9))
 (segment (start 54.75 71.0576) (end 54.75 74.55) (width 0.25) (layer F.Cu) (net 9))
 (segment (start 54.75 74.55) (end 55.238001 75.038001) (width 0.25) (layer F.Cu) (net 9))
 (segment (start 55.238001 75.038001) (end 56 75.8) (width 0.25) (layer F.Cu) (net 9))
 (segment (start 57.4563 69.9513) (end 57.4563 72.1863) (width 0.25) (layer F.Cu) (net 10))
 (segment (start 57.4563 72.1863) (end 58.53 73.26) (width 0.25) (layer F.Cu) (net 10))
 (segment (start 56 73.3) (end 58.49 73.3) (width 0.25) (layer F.Cu) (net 10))
 (segment (start 58.49 73.3) (end 58.53 73.26) (width 0.25) (layer F.Cu) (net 10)))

